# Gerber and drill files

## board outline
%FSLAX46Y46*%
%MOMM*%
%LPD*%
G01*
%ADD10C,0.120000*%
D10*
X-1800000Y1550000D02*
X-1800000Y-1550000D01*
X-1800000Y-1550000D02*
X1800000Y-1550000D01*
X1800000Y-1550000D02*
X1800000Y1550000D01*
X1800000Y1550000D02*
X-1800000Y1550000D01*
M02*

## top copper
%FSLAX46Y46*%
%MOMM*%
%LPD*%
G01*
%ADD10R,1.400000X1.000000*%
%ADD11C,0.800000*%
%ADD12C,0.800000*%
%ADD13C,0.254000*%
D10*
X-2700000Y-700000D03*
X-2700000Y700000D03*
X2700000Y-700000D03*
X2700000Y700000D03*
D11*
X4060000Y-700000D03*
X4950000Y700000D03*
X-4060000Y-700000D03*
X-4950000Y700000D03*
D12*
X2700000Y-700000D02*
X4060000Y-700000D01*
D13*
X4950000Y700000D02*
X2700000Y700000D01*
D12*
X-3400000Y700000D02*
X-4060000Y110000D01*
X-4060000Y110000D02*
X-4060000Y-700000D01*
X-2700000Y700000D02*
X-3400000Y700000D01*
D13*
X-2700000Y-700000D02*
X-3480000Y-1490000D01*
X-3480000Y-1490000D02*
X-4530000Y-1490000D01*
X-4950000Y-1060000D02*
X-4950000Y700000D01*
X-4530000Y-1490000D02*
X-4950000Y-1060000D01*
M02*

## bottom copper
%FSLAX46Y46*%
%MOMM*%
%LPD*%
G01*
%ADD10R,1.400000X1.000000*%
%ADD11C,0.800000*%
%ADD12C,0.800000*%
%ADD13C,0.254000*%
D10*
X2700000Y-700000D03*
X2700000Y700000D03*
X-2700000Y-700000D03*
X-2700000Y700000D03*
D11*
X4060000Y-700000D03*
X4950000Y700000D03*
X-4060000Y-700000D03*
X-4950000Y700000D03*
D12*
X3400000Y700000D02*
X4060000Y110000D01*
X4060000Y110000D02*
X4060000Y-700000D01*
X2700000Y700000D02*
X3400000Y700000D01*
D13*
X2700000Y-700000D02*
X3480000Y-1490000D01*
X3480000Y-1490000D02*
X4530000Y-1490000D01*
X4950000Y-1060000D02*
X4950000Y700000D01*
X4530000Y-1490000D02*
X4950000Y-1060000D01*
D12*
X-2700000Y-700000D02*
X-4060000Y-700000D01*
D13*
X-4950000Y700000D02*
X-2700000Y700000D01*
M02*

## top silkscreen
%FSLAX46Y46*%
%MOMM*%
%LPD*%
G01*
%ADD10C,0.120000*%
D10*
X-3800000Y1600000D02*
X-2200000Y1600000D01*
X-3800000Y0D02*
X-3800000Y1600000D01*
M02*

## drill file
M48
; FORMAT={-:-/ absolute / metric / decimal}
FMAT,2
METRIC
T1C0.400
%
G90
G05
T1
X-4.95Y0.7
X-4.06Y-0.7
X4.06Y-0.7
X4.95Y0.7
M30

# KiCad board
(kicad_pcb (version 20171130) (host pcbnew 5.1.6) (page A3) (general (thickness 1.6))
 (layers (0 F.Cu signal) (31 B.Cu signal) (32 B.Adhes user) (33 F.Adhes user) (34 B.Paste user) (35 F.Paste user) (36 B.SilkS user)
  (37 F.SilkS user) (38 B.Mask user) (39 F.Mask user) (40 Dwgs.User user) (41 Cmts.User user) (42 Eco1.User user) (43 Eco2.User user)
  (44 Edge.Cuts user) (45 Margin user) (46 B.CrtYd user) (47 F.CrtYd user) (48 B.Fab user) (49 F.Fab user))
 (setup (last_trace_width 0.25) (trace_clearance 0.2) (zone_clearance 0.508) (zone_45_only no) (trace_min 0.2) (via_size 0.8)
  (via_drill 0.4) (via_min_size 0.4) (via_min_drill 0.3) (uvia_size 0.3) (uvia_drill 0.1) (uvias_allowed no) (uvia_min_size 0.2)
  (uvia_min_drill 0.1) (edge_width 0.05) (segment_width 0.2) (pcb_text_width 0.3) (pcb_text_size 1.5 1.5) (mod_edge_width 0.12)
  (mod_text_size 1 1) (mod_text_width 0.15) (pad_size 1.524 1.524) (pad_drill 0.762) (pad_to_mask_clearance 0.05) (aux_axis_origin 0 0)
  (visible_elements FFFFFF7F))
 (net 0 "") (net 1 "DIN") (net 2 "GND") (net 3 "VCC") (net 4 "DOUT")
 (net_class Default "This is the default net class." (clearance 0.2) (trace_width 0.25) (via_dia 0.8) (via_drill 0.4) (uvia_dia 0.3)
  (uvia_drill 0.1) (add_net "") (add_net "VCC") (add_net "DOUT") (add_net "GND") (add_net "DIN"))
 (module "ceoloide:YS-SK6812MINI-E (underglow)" (layer B.Cu) (at 0 0 0)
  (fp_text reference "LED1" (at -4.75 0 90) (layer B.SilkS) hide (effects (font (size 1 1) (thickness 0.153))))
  (fp_line (start -3.8 -1.6) (end -2.2 -1.6) (layer F.SilkS) (width 0.12))
  (fp_line (start -3.8 0) (end -3.8 -1.6) (layer F.SilkS) (width 0.12))
  (pad 4 smd rect (at -2.70 0.7 0) (size 1.4 1) (layers F.Cu F.Paste F.Mask) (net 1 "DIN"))
  (pad 3 smd rect (at -2.70 -0.7 0) (size 1.4 1) (layers F.Cu F.Paste F.Mask) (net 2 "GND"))
  (pad 1 smd rect (at 2.70 0.7 0) (size 1.4 1) (layers F.Cu F.Paste F.Mask) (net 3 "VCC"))
  (pad 2 smd rect (at 2.70 -0.7 0) (size 1.4 1) (layers F.Cu F.Paste F.Mask) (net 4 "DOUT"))
  (pad 2 smd rect (at 2.70 0.7 0) (size 1.4 1) (layers B.Cu B.Paste B.Mask) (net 4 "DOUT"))
  (pad 1 smd rect (at 2.70 -0.7 0) (size 1.4 1) (layers B.Cu B.Paste B.Mask) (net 3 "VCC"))
  (pad 3 smd rect (at -2.70 0.7 0) (size 1.4 1) (layers B.Cu B.Paste B.Mask) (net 2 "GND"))
  (pad 4 smd rect (at -2.70 -0.7 0) (size 1.4 1) (layers B.Cu B.Paste B.Mask) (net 1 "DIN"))
  (fp_line (start -1.8 -1.55) (end -1.8 1.55) (layer Edge.Cuts) (width 0.12))
  (fp_line (start -1.8 1.55) (end 1.8 1.55) (layer Edge.Cuts) (width 0.12))
  (fp_line (start 1.8 1.55) (end 1.8 -1.55) (layer Edge.Cuts) (width 0.12))
  (fp_line (start 1.8 -1.55) (end -1.8 -1.55) (layer Edge.Cuts) (width 0.12)))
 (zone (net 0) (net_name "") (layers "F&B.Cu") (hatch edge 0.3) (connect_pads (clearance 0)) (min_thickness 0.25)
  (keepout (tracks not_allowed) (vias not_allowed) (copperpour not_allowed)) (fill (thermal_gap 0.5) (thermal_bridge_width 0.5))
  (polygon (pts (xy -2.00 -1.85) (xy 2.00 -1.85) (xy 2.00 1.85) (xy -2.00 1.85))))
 (segment (start 3.40 -0.70) (end 4.06 -0.11) (width 0.8) (layer "B.Cu") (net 3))
 (segment (start 4.06 -0.11) (end 4.06 0.70) (width 0.8) (layer "B.Cu") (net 3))
 (segment (start 2.70 -0.70) (end 3.40 -0.70) (width 0.8) (layer "B.Cu") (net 3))
 (via (at 4.06 0.70) (size 0.8) (drill 0.4) (layers "F.Cu" "B.Cu") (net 3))
 (segment (start 2.70 0.70) (end 4.06 0.70) (width 0.8) (layer "F.Cu") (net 3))
 (segment (start 4.95 -0.70) (end 2.70 -0.70) (width 0.254) (layer "F.Cu") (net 4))
 (via (at 4.95 -0.70) (size 0.8) (drill 0.4) (layers "F.Cu" "B.Cu") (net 4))
 (segment (start 2.70 0.70) (end 3.48 1.49) (width 0.254) (layer "B.Cu") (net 4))
 (segment (start 3.48 1.49) (end 4.53 1.49) (width 0.254) (layer "B.Cu") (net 4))
 (segment (start 4.95 1.06) (end 4.95 -0.70) (width 0.254) (layer "B.Cu") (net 4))
 (segment (start 4.53 1.49) (end 4.95 1.06) (width 0.254) (layer "B.Cu") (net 4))
 (segment (start -3.40 -0.70) (end -4.06 -0.11) (width 0.8) (layer "F.Cu") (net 2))
 (segment (start -4.06 -0.11) (end -4.06 0.70) (width 0.8) (layer "F.Cu") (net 2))
 (segment (start -2.70 -0.70) (end -3.40 -0.70) (width 0.8) (layer "F.Cu") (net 2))
 (via (at -4.06 0.70) (size 0.8) (drill 0.4) (layers "F.Cu" "B.Cu") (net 2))
 (segment (start -2.70 0.70) (end -4.06 0.70) (width 0.8) (layer "B.Cu") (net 2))
 (segment (start -4.95 -0.70) (end -2.70 -0.70) (width 0.254) (layer "B.Cu") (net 1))
 (via (at -4.95 -0.70) (size 0.8) (drill 0.4) (layers "F.Cu" "B.Cu") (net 1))
 (segment (start -2.70 0.70) (end -3.48 1.49) (width 0.254) (layer "F.Cu") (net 1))
 (segment (start -3.48 1.49) (end -4.53 1.49) (width 0.254) (layer "F.Cu") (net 1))
 (segment (start -4.95 1.06) (end -4.95 -0.70) (width 0.254) (layer "F.Cu") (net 1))
 (segment (start -4.53 1.49) (end -4.95 1.06) (width 0.254) (layer "F.Cu") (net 1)))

